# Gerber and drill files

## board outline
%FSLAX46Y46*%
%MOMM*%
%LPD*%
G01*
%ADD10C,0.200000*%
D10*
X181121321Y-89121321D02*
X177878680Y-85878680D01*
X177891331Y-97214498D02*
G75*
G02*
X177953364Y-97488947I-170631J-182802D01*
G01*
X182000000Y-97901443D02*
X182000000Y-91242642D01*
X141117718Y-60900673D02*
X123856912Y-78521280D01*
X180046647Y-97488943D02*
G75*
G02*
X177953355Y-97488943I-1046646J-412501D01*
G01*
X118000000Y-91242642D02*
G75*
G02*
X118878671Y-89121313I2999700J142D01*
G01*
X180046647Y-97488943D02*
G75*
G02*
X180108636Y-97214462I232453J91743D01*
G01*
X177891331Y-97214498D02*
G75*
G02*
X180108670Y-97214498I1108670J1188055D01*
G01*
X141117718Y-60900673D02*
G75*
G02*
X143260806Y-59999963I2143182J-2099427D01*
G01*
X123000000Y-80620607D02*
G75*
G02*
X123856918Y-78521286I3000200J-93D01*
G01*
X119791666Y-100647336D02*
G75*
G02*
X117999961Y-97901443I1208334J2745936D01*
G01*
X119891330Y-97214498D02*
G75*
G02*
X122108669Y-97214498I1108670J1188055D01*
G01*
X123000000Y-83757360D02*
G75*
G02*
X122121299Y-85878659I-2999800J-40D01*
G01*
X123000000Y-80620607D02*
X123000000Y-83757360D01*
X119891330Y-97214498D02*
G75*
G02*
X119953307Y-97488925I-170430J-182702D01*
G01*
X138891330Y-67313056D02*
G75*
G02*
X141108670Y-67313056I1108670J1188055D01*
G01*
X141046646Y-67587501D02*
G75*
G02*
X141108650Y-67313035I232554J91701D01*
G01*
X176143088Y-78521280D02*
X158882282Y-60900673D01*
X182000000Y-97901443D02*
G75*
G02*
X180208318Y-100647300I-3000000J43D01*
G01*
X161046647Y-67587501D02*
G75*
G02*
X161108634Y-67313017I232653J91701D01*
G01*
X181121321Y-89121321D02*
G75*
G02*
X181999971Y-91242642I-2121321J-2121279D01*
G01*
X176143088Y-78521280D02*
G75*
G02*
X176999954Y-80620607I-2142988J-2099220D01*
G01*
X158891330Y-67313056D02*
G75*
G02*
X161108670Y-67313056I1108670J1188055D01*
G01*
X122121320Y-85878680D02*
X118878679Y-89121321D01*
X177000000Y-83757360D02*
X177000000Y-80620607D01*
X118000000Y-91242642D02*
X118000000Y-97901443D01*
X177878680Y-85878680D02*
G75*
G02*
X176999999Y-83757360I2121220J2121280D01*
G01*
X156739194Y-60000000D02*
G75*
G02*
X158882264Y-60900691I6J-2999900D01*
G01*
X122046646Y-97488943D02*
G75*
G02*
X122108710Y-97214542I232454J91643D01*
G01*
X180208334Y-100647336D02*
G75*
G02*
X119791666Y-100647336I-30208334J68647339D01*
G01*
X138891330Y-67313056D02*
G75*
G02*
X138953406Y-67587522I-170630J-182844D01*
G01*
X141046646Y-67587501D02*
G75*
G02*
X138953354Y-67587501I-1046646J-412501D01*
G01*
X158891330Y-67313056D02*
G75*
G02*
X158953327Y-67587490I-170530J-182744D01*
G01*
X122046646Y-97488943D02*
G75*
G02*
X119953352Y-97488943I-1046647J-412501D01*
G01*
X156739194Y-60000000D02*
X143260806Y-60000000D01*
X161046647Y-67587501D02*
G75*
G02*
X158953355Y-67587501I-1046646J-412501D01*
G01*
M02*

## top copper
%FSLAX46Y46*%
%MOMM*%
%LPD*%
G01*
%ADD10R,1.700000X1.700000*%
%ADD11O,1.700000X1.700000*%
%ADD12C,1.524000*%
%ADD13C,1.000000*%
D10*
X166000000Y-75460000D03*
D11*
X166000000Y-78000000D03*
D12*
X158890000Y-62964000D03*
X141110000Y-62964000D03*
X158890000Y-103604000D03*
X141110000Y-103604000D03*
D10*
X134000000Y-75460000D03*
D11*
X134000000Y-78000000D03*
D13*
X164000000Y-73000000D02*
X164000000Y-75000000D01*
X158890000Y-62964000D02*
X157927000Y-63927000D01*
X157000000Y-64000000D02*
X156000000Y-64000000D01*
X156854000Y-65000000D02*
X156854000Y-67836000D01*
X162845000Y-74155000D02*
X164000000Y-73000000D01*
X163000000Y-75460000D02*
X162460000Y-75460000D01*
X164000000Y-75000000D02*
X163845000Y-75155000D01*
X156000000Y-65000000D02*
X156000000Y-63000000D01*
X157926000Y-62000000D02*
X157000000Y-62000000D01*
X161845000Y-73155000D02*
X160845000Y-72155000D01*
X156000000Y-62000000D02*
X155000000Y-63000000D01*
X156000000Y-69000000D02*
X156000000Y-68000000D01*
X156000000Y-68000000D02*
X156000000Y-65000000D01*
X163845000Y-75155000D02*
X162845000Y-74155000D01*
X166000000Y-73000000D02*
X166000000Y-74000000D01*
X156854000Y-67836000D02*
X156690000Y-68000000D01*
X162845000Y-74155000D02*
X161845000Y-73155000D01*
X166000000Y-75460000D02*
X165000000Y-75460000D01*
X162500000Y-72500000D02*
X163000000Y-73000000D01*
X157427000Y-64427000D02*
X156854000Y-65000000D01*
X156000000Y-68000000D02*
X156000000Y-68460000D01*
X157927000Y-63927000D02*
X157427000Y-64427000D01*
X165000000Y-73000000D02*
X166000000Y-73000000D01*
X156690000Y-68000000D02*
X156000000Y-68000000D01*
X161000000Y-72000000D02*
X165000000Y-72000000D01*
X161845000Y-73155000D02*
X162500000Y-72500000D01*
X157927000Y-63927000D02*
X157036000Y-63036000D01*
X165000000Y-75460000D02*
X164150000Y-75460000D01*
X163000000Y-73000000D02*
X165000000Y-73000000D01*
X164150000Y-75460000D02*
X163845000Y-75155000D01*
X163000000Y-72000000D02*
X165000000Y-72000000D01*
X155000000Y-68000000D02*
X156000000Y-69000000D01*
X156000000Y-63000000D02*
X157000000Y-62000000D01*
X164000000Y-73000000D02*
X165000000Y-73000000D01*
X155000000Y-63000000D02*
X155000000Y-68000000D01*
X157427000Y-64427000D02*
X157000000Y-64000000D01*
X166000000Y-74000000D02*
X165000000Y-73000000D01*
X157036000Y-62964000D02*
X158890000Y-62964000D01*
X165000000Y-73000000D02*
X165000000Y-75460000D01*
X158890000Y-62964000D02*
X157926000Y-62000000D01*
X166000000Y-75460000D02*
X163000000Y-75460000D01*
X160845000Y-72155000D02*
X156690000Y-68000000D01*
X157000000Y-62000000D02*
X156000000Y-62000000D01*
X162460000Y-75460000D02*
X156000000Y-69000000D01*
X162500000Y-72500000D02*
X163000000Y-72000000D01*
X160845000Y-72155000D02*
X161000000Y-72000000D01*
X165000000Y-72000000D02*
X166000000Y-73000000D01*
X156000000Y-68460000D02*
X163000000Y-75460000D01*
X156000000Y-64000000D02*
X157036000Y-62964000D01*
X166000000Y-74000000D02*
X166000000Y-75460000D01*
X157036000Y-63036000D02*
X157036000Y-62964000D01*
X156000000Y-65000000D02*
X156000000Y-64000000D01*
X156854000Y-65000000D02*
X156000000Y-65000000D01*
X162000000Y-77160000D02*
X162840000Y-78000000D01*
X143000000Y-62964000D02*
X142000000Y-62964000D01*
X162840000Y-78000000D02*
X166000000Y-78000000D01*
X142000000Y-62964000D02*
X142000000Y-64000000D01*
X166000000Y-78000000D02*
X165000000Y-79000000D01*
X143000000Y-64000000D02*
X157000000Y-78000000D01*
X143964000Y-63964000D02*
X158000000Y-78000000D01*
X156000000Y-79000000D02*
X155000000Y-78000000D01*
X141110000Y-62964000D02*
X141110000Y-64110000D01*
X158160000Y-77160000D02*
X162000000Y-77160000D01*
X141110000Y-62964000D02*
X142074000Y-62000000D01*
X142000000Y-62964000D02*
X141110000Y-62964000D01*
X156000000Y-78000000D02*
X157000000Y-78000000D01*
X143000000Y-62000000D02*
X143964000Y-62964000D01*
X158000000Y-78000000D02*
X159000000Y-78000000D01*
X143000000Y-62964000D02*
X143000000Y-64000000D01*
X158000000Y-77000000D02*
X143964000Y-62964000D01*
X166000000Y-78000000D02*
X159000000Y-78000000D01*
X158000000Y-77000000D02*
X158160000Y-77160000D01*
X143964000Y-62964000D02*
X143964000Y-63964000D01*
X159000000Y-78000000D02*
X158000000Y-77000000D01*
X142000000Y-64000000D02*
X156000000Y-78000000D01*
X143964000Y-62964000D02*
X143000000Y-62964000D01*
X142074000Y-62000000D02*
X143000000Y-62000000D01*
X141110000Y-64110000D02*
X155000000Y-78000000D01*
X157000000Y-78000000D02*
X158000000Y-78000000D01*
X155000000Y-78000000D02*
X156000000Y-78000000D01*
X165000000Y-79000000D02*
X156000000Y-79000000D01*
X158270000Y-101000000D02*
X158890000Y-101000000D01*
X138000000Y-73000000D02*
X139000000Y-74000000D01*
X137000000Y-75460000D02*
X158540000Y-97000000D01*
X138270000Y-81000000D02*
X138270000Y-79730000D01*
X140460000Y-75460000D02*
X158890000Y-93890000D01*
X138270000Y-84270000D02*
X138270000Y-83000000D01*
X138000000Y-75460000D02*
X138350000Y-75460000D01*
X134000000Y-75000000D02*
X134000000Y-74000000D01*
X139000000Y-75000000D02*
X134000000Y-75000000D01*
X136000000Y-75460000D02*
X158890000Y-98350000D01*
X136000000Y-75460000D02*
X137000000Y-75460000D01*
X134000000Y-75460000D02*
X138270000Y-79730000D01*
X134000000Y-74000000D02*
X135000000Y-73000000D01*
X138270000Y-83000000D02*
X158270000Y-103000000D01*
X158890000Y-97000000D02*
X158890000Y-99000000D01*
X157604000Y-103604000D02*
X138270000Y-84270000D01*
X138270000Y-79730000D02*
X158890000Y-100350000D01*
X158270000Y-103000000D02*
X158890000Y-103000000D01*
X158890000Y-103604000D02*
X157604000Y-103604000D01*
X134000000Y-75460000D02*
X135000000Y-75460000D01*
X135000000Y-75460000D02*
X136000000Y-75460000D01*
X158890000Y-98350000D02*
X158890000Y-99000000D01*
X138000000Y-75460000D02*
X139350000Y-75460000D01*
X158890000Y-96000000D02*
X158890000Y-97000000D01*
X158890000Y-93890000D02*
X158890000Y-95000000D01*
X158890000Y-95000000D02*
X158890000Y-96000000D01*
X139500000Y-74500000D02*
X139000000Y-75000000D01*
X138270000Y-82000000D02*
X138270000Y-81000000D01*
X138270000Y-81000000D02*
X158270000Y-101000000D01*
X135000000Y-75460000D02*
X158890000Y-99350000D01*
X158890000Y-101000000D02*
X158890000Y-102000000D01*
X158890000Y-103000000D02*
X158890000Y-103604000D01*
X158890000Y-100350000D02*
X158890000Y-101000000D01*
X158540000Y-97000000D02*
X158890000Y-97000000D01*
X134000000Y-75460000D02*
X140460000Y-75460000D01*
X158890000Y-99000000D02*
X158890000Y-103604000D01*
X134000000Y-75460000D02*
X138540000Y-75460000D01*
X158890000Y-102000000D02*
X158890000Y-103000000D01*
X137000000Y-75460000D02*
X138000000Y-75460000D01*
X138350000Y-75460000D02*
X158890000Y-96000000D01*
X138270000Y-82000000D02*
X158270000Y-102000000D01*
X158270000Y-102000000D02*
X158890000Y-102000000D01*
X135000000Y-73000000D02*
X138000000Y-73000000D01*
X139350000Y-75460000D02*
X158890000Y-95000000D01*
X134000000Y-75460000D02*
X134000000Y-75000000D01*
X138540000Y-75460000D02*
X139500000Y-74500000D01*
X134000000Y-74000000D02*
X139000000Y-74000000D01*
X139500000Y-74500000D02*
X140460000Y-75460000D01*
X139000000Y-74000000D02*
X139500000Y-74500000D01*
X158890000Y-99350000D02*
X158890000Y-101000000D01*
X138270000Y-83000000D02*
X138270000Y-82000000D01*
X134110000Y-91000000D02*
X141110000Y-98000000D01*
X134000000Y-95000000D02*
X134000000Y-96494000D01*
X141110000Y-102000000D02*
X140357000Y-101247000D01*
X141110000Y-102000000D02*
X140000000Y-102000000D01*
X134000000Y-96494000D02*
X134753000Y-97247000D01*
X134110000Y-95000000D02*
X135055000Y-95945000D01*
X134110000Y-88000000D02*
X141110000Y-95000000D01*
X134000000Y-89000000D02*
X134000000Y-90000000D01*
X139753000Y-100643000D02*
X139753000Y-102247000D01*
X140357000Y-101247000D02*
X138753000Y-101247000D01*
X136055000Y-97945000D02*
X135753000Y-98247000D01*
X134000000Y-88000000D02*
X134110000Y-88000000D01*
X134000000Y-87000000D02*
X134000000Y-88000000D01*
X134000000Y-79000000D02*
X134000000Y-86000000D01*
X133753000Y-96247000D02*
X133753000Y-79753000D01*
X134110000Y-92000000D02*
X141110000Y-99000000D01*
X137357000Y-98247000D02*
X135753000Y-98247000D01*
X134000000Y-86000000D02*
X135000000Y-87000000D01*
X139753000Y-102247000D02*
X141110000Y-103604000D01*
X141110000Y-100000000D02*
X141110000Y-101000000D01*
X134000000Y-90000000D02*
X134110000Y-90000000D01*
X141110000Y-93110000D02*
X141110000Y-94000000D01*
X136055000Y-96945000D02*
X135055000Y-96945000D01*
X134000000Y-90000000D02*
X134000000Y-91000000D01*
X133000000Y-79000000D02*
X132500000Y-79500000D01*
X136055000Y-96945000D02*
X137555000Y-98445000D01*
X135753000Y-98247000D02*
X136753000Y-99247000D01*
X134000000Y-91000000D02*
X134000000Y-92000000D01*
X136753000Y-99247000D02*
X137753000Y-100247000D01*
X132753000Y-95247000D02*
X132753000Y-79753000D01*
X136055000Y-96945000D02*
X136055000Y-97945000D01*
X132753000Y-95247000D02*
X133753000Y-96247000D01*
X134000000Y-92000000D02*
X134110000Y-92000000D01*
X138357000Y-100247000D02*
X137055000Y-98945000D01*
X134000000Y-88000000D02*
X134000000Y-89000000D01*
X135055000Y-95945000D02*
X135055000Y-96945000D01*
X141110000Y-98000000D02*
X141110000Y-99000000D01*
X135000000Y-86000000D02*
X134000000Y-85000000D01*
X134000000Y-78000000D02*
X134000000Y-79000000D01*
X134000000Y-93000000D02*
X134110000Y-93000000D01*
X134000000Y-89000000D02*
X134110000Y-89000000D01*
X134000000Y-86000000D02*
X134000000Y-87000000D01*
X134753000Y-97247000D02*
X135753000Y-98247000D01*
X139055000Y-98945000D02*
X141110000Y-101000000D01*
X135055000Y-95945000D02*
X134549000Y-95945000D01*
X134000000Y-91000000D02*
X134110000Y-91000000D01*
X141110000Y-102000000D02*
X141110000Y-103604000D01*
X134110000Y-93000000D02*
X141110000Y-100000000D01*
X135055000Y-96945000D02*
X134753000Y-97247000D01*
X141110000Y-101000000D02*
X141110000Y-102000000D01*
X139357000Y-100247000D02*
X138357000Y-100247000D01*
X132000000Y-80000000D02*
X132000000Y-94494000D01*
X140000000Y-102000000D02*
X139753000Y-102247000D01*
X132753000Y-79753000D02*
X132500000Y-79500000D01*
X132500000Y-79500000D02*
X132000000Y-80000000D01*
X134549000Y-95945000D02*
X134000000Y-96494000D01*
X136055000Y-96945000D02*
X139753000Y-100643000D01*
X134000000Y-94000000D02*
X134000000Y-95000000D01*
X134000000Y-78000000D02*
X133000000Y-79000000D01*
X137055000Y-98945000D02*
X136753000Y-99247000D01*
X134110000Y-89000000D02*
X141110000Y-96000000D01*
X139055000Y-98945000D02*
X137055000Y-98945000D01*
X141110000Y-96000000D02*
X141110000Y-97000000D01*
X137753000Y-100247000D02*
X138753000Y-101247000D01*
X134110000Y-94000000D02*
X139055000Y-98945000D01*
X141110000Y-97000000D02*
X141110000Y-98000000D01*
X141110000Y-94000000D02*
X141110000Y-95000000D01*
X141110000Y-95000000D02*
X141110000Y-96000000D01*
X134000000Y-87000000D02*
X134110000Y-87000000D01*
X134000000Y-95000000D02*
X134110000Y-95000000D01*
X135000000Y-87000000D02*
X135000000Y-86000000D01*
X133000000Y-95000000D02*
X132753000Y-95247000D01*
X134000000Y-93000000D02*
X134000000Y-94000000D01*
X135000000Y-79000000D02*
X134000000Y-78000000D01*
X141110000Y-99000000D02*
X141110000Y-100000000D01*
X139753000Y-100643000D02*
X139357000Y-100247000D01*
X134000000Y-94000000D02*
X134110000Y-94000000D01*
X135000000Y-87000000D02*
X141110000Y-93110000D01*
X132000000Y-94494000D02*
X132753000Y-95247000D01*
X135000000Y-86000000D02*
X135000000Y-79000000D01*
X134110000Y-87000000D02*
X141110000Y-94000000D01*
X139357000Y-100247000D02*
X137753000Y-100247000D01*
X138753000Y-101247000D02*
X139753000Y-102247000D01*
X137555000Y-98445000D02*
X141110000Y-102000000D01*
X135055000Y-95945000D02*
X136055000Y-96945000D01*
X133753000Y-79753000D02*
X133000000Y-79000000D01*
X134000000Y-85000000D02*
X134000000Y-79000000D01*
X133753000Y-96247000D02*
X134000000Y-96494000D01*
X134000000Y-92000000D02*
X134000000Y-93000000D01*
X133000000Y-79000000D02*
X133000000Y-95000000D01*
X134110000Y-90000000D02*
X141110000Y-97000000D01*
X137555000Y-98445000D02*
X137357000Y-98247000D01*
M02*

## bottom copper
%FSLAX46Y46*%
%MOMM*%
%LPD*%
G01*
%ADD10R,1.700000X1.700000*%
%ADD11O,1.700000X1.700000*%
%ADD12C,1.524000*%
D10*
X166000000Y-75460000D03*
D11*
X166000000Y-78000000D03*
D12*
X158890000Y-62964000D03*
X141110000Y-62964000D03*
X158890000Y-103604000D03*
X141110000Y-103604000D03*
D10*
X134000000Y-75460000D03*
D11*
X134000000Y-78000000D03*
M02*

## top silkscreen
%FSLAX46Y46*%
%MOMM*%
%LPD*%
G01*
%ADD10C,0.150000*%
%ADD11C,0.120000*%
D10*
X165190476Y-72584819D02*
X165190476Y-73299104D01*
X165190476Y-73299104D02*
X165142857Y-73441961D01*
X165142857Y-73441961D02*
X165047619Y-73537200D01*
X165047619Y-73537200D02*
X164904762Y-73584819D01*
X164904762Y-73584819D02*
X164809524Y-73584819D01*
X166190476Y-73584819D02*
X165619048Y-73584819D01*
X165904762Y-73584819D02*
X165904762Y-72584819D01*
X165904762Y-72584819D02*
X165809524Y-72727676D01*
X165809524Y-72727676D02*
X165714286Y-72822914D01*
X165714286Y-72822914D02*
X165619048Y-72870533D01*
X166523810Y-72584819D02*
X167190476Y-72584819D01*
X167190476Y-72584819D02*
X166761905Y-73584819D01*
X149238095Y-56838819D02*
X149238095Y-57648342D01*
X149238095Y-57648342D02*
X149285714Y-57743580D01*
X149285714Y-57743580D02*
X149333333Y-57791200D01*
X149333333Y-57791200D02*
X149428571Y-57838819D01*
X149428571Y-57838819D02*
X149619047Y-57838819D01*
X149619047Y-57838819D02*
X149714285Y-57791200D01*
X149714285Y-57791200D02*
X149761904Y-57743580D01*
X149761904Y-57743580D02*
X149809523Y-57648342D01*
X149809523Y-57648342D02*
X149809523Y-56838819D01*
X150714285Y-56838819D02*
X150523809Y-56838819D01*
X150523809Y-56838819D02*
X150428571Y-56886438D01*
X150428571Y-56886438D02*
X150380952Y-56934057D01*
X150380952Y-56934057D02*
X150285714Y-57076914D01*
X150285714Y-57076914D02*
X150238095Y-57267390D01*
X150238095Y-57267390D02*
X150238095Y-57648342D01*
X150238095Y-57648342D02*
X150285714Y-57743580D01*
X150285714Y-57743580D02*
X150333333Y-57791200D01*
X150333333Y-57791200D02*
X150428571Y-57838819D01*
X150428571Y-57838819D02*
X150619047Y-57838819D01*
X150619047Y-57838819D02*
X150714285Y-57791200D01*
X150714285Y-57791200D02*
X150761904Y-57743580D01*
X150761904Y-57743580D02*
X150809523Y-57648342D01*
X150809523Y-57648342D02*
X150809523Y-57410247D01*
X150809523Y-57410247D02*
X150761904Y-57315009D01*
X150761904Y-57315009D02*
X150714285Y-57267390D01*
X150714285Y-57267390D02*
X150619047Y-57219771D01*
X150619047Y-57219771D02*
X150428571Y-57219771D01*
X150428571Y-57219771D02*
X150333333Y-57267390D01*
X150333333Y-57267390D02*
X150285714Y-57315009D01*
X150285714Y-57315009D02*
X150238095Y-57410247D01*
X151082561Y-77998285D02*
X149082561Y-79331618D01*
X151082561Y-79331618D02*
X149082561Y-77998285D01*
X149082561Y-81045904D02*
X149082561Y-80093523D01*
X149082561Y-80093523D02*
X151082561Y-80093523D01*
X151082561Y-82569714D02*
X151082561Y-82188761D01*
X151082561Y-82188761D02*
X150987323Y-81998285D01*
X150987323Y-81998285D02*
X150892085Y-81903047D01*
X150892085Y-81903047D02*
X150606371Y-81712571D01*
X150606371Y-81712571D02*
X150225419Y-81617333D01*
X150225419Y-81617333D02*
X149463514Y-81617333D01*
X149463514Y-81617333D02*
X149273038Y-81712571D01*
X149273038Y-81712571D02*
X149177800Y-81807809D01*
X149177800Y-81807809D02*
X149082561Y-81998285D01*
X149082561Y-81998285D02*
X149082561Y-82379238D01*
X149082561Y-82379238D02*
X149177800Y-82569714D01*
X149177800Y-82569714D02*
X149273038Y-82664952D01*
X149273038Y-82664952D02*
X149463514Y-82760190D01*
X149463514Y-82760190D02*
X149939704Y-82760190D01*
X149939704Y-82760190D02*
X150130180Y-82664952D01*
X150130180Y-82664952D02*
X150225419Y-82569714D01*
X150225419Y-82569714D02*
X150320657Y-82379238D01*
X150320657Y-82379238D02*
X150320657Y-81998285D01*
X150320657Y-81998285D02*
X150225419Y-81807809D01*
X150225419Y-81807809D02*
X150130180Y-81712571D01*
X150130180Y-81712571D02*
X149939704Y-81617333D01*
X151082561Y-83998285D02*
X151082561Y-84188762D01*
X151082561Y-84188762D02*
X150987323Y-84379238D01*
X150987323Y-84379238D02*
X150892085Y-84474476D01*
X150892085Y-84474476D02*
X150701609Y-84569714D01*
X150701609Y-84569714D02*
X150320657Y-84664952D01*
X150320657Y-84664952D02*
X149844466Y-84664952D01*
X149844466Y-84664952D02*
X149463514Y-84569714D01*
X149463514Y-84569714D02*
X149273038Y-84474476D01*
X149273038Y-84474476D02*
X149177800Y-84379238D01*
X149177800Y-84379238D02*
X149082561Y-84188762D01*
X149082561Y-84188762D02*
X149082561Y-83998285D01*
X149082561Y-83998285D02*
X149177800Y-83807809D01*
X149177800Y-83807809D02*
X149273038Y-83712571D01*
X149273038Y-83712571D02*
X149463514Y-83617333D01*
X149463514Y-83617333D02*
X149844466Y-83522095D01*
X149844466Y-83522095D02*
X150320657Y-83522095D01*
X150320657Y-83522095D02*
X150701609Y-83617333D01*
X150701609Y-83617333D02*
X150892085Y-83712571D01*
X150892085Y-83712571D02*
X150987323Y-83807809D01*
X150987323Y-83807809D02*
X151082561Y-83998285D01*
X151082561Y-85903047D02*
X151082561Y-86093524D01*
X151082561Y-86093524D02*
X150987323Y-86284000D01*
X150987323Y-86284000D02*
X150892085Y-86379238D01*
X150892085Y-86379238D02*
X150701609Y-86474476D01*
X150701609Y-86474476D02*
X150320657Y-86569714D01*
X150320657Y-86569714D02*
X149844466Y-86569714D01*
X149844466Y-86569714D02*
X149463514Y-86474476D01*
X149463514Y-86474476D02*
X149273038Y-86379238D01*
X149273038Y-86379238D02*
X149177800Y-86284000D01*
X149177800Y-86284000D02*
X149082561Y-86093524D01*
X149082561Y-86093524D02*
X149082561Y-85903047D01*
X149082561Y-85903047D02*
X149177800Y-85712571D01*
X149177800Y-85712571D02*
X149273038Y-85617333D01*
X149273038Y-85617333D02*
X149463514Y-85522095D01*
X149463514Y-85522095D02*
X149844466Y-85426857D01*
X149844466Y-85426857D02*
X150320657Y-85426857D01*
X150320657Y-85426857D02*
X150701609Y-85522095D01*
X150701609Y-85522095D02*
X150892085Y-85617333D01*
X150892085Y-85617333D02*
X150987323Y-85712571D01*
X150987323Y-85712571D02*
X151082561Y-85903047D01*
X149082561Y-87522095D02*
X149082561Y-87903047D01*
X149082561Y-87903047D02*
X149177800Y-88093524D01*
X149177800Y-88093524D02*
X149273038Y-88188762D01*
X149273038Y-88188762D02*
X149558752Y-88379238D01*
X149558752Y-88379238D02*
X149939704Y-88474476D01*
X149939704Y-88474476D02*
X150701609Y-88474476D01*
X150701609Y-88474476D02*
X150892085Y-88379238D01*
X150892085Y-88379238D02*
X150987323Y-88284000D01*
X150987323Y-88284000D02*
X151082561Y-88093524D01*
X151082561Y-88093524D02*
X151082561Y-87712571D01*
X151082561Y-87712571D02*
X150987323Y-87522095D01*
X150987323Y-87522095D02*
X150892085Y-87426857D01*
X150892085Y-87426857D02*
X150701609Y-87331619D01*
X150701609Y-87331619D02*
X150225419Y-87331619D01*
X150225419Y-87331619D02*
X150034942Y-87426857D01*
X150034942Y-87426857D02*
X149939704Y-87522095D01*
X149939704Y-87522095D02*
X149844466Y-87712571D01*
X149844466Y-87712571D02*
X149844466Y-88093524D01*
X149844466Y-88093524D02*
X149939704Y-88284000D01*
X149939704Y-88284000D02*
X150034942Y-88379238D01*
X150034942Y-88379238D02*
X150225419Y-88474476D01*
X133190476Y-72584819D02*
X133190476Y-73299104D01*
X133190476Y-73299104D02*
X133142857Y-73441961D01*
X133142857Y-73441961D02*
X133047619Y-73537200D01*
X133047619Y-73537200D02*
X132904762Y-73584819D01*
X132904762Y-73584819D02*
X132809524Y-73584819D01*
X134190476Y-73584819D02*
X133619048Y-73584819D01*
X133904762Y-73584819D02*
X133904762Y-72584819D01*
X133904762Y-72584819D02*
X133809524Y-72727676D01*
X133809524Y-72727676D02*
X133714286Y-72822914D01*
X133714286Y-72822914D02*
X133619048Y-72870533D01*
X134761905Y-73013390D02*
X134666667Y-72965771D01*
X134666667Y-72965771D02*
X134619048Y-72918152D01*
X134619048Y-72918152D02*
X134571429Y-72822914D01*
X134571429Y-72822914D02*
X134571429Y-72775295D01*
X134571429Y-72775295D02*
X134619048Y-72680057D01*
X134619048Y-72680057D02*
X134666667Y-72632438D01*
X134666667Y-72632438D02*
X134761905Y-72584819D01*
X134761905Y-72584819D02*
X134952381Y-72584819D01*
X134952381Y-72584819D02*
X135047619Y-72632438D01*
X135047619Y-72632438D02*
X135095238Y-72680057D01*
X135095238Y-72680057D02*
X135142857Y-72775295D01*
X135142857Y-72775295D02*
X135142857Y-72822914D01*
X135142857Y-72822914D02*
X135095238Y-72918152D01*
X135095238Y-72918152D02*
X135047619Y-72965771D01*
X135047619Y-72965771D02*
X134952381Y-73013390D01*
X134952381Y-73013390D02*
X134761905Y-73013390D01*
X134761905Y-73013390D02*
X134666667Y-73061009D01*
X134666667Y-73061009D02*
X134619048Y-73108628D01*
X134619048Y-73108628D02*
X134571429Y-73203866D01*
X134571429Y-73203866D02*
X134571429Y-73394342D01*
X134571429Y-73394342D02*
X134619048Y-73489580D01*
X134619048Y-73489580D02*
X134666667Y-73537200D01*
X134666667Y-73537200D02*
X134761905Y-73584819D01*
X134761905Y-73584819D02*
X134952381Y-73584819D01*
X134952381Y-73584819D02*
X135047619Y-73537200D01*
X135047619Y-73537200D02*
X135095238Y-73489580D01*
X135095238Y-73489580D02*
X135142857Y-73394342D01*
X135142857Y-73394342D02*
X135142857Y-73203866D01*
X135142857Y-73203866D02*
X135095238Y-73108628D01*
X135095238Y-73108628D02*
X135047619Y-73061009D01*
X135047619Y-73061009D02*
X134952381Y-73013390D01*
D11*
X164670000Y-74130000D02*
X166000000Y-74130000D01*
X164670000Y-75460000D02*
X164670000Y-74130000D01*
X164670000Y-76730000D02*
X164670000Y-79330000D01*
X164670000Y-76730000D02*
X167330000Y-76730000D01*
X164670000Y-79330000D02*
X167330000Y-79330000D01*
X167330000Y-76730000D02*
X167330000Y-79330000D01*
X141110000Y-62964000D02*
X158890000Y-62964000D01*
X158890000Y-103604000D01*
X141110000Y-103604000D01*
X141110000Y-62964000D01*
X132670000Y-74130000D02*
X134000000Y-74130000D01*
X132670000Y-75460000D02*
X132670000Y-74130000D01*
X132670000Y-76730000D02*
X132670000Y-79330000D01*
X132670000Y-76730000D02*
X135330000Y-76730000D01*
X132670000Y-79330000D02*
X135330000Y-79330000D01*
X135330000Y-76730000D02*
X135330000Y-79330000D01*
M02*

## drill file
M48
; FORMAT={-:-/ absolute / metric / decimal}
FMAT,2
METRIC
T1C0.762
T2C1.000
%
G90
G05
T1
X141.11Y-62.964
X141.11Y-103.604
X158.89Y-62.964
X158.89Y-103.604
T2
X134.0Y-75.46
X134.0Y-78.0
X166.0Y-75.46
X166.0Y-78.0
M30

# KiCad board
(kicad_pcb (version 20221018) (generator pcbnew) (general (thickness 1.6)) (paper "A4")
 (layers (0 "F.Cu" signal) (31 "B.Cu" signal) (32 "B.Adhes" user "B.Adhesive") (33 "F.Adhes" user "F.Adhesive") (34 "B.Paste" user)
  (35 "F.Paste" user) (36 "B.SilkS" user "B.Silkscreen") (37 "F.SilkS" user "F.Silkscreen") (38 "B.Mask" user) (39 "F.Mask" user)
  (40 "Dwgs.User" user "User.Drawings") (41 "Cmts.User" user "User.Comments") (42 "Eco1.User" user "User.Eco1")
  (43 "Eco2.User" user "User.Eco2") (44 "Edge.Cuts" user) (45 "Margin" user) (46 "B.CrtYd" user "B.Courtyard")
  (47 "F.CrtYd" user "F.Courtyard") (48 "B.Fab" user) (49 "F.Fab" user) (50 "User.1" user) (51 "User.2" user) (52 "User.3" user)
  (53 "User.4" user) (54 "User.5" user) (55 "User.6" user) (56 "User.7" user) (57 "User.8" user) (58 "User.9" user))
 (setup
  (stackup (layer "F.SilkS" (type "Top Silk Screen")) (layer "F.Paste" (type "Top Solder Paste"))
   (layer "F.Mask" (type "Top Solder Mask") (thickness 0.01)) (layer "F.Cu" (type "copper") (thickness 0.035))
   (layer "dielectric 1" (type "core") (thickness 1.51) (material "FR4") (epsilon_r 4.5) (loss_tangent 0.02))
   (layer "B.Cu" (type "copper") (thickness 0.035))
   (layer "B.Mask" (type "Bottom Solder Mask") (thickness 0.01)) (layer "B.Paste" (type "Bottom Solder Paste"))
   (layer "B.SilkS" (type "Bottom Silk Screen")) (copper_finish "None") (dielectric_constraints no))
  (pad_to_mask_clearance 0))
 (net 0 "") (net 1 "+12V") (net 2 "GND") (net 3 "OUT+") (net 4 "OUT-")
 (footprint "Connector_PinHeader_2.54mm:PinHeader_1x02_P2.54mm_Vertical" (layer "F.Cu") (at 166 75.46)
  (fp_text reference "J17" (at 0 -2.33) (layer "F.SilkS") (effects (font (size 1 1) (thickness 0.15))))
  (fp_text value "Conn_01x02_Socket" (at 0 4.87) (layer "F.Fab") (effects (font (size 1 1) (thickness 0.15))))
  (fp_line (start -1.33 -1.33) (end 0 -1.33) (stroke (width 0.12) (type solid)) (layer "F.SilkS"))
  (fp_line (start -1.33 0) (end -1.33 -1.33) (stroke (width 0.12) (type solid)) (layer "F.SilkS"))
  (fp_line (start -1.33 1.27) (end -1.33 3.87) (stroke (width 0.12) (type solid)) (layer "F.SilkS"))
  (fp_line (start -1.33 1.27) (end 1.33 1.27) (stroke (width 0.12) (type solid)) (layer "F.SilkS"))
  (fp_line (start -1.33 3.87) (end 1.33 3.87) (stroke (width 0.12) (type solid)) (layer "F.SilkS"))
  (fp_line (start 1.33 1.27) (end 1.33 3.87) (stroke (width 0.12) (type solid)) (layer "F.SilkS"))
  (pad "1" thru_hole rect (at 0 0) (size 1.7 1.7) (drill 1) (layers "*.Cu" "*.Mask") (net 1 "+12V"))
  (pad "2" thru_hole oval (at 0 2.54) (size 1.7 1.7) (drill 1) (layers "*.Cu" "*.Mask") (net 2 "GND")))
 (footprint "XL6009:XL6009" (layer "F.Cu") (at 150 57.884)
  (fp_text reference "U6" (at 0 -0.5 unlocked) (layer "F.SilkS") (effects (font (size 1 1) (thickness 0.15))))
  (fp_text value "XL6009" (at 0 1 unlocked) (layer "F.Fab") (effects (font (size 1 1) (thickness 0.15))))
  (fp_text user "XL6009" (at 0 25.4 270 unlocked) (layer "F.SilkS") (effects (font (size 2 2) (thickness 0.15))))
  (fp_rect (start -8.89 5.08) (end 8.89 45.72) (stroke (width 0.12) (type solid)) (fill none) (layer "F.SilkS"))
  (pad "1" thru_hole circle (at 8.89 5.08) (size 1.524 1.524) (drill 0.762) (layers "*.Cu" "*.Mask") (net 1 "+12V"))
  (pad "2" thru_hole circle (at -8.89 5.08) (size 1.524 1.524) (drill 0.762) (layers "*.Cu" "*.Mask") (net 2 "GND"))
  (pad "3" thru_hole circle (at 8.89 45.72) (size 1.524 1.524) (drill 0.762) (layers "*.Cu" "*.Mask") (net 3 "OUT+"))
  (pad "4" thru_hole circle (at -8.89 45.72) (size 1.524 1.524) (drill 0.762) (layers "*.Cu" "*.Mask") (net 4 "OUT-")))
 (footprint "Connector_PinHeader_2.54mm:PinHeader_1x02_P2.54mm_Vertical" (layer "F.Cu") (at 134 75.46)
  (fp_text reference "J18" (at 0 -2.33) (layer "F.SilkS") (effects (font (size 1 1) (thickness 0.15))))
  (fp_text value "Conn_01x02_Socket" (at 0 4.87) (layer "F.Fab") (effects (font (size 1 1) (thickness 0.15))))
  (fp_line (start -1.33 -1.33) (end 0 -1.33) (stroke (width 0.12) (type solid)) (layer "F.SilkS"))
  (fp_line (start -1.33 0) (end -1.33 -1.33) (stroke (width 0.12) (type solid)) (layer "F.SilkS"))
  (fp_line (start -1.33 1.27) (end -1.33 3.87) (stroke (width 0.12) (type solid)) (layer "F.SilkS"))
  (fp_line (start -1.33 1.27) (end 1.33 1.27) (stroke (width 0.12) (type solid)) (layer "F.SilkS"))
  (fp_line (start -1.33 3.87) (end 1.33 3.87) (stroke (width 0.12) (type solid)) (layer "F.SilkS"))
  (fp_line (start 1.33 1.27) (end 1.33 3.87) (stroke (width 0.12) (type solid)) (layer "F.SilkS"))
  (pad "1" thru_hole rect (at 0 0) (size 1.7 1.7) (drill 1) (layers "*.Cu" "*.Mask") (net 3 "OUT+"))
  (pad "2" thru_hole oval (at 0 2.54) (size 1.7 1.7) (drill 1) (layers "*.Cu" "*.Mask") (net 4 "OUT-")))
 (gr_line (start 181.121321 89.121321) (end 177.87868 85.87868) (stroke (width 0.2) (type solid)) (layer "Edge.Cuts"))
 (gr_arc (start 177.891331 97.214498) (mid 177.964609 97.342164) (end 177.953354 97.488943) (stroke (width 0.2) (type solid))
  (layer "Edge.Cuts"))
 (gr_line (start 182 97.901443) (end 182 91.242642) (stroke (width 0.2) (type solid)) (layer "Edge.Cuts"))
 (gr_line (start 141.117718 60.900673) (end 123.856912 78.52128) (stroke (width 0.2) (type solid)) (layer "Edge.Cuts"))
 (gr_arc (start 180.046647 97.488943) (mid 179 99.026444) (end 177.953354 97.488943) (stroke (width 0.2) (type solid)) (layer "Edge.Cuts"))
 (gr_arc (start 118 91.242642) (mid 118.228341 90.094582) (end 118.878679 89.121321) (stroke (width 0.2) (type solid)) (layer "Edge.Cuts"))
 (gr_arc (start 180.046647 97.488943) (mid 180.035365 97.342158) (end 180.10867 97.214498) (stroke (width 0.2) (type solid))
  (layer "Edge.Cuts"))
 (gr_arc (start 177.891331 97.214498) (mid 179 94.401444) (end 180.10867 97.214498) (stroke (width 0.2) (type solid)) (layer "Edge.Cuts"))
 (gr_arc (start 141.117718 60.900673) (mid 142.09848 60.23433) (end 143.260806 60) (stroke (width 0.2) (type solid)) (layer "Edge.Cuts"))
 (gr_arc (start 123 80.620607) (mid 123.222489 79.486874) (end 123.856912 78.52128) (stroke (width 0.2) (type solid)) (layer "Edge.Cuts"))
 (gr_arc (start 119.791666 100.647336) (mid 118.487531 99.540802) (end 118 97.901443) (stroke (width 0.2) (type solid)) (layer "Edge.Cuts"))
 (gr_arc (start 119.89133 97.214498) (mid 120.999999 94.401444) (end 122.108669 97.214498) (stroke (width 0.2) (type solid))
  (layer "Edge.Cuts"))
 (gr_arc (start 123 83.75736) (mid 122.771654 84.905417) (end 122.12132 85.87868) (stroke (width 0.2) (type solid)) (layer "Edge.Cuts"))
 (gr_line (start 123 80.620607) (end 123 83.75736) (stroke (width 0.2) (type solid)) (layer "Edge.Cuts"))
 (gr_arc (start 119.89133 97.214498) (mid 119.964638 97.342161) (end 119.953353 97.488943) (stroke (width 0.2) (type solid))
  (layer "Edge.Cuts"))
 (gr_arc (start 138.89133 67.313056) (mid 140 64.500001) (end 141.10867 67.313056) (stroke (width 0.2) (type solid)) (layer "Edge.Cuts"))
 (gr_arc (start 141.046646 67.587501) (mid 141.035382 67.440731) (end 141.10867 67.313056) (stroke (width 0.2) (type solid))
  (layer "Edge.Cuts"))
 (gr_line (start 176.143088 78.52128) (end 158.882282 60.900673) (stroke (width 0.2) (type solid)) (layer "Edge.Cuts"))
 (gr_arc (start 182 97.901443) (mid 181.512469 99.540802) (end 180.208334 100.647336) (stroke (width 0.2) (type solid)) (layer "Edge.Cuts"))
 (gr_arc (start 161.046647 67.587501) (mid 161.035388 67.440729) (end 161.10867 67.313056) (stroke (width 0.2) (type solid))
  (layer "Edge.Cuts"))
 (gr_arc (start 181.121321 89.121321) (mid 181.77164 90.094591) (end 182 91.242642) (stroke (width 0.2) (type solid)) (layer "Edge.Cuts"))
 (gr_arc (start 176.143088 78.52128) (mid 176.777534 79.486864) (end 177 80.620607) (stroke (width 0.2) (type solid)) (layer "Edge.Cuts"))
 (gr_arc (start 158.89133 67.313056) (mid 160 64.500001) (end 161.10867 67.313056) (stroke (width 0.2) (type solid)) (layer "Edge.Cuts"))
 (gr_line (start 122.12132 85.87868) (end 118.878679 89.121321) (stroke (width 0.2) (type solid)) (layer "Edge.Cuts"))
 (gr_line (start 177 83.75736) (end 177 80.620607) (stroke (width 0.2) (type solid)) (layer "Edge.Cuts"))
 (gr_line (start 118 91.242642) (end 118 97.901443) (stroke (width 0.2) (type solid)) (layer "Edge.Cuts"))
 (gr_arc (start 177.87868 85.87868) (mid 177.228356 84.905411) (end 177 83.75736) (stroke (width 0.2) (type solid)) (layer "Edge.Cuts"))
 (gr_arc (start 156.739194 60) (mid 157.901527 60.234315) (end 158.882282 60.900673) (stroke (width 0.2) (type solid)) (layer "Edge.Cuts"))
 (gr_arc (start 122.046646 97.488943) (mid 122.035369 97.342155) (end 122.108669 97.214498) (stroke (width 0.2) (type solid))
  (layer "Edge.Cuts"))
 (gr_arc (start 180.208334 100.647336) (mid 150 107.000001) (end 119.791666 100.647336) (stroke (width 0.2) (type solid))
  (layer "Edge.Cuts"))
 (gr_arc (start 138.89133 67.313056) (mid 138.964601 67.440727) (end 138.953353 67.587501) (stroke (width 0.2) (type solid))
  (layer "Edge.Cuts"))
 (gr_arc (start 141.046646 67.587501) (mid 139.999999 69.125003) (end 138.953353 67.587501) (stroke (width 0.2) (type solid))
  (layer "Edge.Cuts"))
 (gr_arc (start 158.89133 67.313056) (mid 158.964631 67.440724) (end 158.953354 67.587501) (stroke (width 0.2) (type solid))
  (layer "Edge.Cuts"))
 (gr_arc (start 122.046646 97.488943) (mid 120.999999 99.026445) (end 119.953353 97.488943) (stroke (width 0.2) (type solid))
  (layer "Edge.Cuts"))
 (gr_line (start 156.739194 60) (end 143.260806 60) (stroke (width 0.2) (type solid)) (layer "Edge.Cuts"))
 (gr_arc (start 161.046647 67.587501) (mid 160 69.125002) (end 158.953354 67.587501) (stroke (width 0.2) (type solid)) (layer "Edge.Cuts"))
 (segment (start 164 73) (end 164 75) (width 1) (layer "F.Cu") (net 1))
 (segment (start 158.89 62.964) (end 157.927 63.927) (width 1) (layer "F.Cu") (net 1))
 (segment (start 157 64) (end 156 64) (width 1) (layer "F.Cu") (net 1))
 (segment (start 156.854 65) (end 156.854 67.836) (width 1) (layer "F.Cu") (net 1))
 (segment (start 162.845 74.155) (end 164 73) (width 1) (layer "F.Cu") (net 1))
 (segment (start 163 75.46) (end 162.46 75.46) (width 1) (layer "F.Cu") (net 1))
 (segment (start 164 75) (end 163.845 75.155) (width 1) (layer "F.Cu") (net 1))
 (segment (start 156 65) (end 156 63) (width 1) (layer "F.Cu") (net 1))
 (segment (start 157.926 62) (end 157 62) (width 1) (layer "F.Cu") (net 1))
 (segment (start 161.845 73.155) (end 160.845 72.155) (width 1) (layer "F.Cu") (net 1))
 (segment (start 156 62) (end 155 63) (width 1) (layer "F.Cu") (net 1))
 (segment (start 156 69) (end 156 68) (width 1) (layer "F.Cu") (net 1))
 (segment (start 156 68) (end 156 65) (width 1) (layer "F.Cu") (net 1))
 (segment (start 163.845 75.155) (end 162.845 74.155) (width 1) (layer "F.Cu") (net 1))
 (segment (start 166 73) (end 166 74) (width 1) (layer "F.Cu") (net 1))
 (segment (start 156.854 67.836) (end 156.69 68) (width 1) (layer "F.Cu") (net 1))
 (segment (start 162.845 74.155) (end 161.845 73.155) (width 1) (layer "F.Cu") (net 1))
 (segment (start 166 75.46) (end 165 75.46) (width 1) (layer "F.Cu") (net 1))
 (segment (start 162.5 72.5) (end 163 73) (width 1) (layer "F.Cu") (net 1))
 (segment (start 157.427 64.427) (end 156.854 65) (width 1) (layer "F.Cu") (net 1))
 (segment (start 156 68) (end 156 68.46) (width 1) (layer "F.Cu") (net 1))
 (segment (start 157.927 63.927) (end 157.427 64.427) (width 1) (layer "F.Cu") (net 1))
 (segment (start 165 73) (end 166 73) (width 1) (layer "F.Cu") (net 1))
 (segment (start 156.69 68) (end 156 68) (width 1) (layer "F.Cu") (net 1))
 (segment (start 161 72) (end 165 72) (width 1) (layer "F.Cu") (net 1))
 (segment (start 161.845 73.155) (end 162.5 72.5) (width 1) (layer "F.Cu") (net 1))
 (segment (start 157.927 63.927) (end 157.036 63.036) (width 1) (layer "F.Cu") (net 1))
 (segment (start 165 75.46) (end 164.15 75.46) (width 1) (layer "F.Cu") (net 1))
 (segment (start 163 73) (end 165 73) (width 1) (layer "F.Cu") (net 1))
 (segment (start 164.15 75.46) (end 163.845 75.155) (width 1) (layer "F.Cu") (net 1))
 (segment (start 163 72) (end 165 72) (width 1) (layer "F.Cu") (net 1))
 (segment (start 155 68) (end 156 69) (width 1) (layer "F.Cu") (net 1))
 (segment (start 156 63) (end 157 62) (width 1) (layer "F.Cu") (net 1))
 (segment (start 164 73) (end 165 73) (width 1) (layer "F.Cu") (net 1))
 (segment (start 155 63) (end 155 68) (width 1) (layer "F.Cu") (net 1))
 (segment (start 157.427 64.427) (end 157 64) (width 1) (layer "F.Cu") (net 1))
 (segment (start 166 74) (end 165 73) (width 1) (layer "F.Cu") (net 1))
 (segment (start 157.036 62.964) (end 158.89 62.964) (width 1) (layer "F.Cu") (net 1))
 (segment (start 165 73) (end 165 75.46) (width 1) (layer "F.Cu") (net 1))
 (segment (start 158.89 62.964) (end 157.926 62) (width 1) (layer "F.Cu") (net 1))
 (segment (start 166 75.46) (end 163 75.46) (width 1) (layer "F.Cu") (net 1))
 (segment (start 160.845 72.155) (end 156.69 68) (width 1) (layer "F.Cu") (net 1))
 (segment (start 157 62) (end 156 62) (width 1) (layer "F.Cu") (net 1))
 (segment (start 162.46 75.46) (end 156 69) (width 1) (layer "F.Cu") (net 1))
 (segment (start 162.5 72.5) (end 163 72) (width 1) (layer "F.Cu") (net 1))
 (segment (start 160.845 72.155) (end 161 72) (width 1) (layer "F.Cu") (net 1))
 (segment (start 165 72) (end 166 73) (width 1) (layer "F.Cu") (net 1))
 (segment (start 156 68.46) (end 163 75.46) (width 1) (layer "F.Cu") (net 1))
 (segment (start 156 64) (end 157.036 62.964) (width 1) (layer "F.Cu") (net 1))
 (segment (start 166 74) (end 166 75.46) (width 1) (layer "F.Cu") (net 1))
 (segment (start 157.036 63.036) (end 157.036 62.964) (width 1) (layer "F.Cu") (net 1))
 (segment (start 156 65) (end 156 64) (width 1) (layer "F.Cu") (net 1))
 (segment (start 156.854 65) (end 156 65) (width 1) (layer "F.Cu") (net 1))
 (segment (start 162 77.16) (end 162.84 78) (width 1) (layer "F.Cu") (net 2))
 (segment (start 143 62.964) (end 142 62.964) (width 1) (layer "F.Cu") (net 2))
 (segment (start 162.84 78) (end 166 78) (width 1) (layer "F.Cu") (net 2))
 (segment (start 142 62.964) (end 142 64) (width 1) (layer "F.Cu") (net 2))
 (segment (start 166 78) (end 165 79) (width 1) (layer "F.Cu") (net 2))
 (segment (start 143 64) (end 157 78) (width 1) (layer "F.Cu") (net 2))
 (segment (start 143.964 63.964) (end 158 78) (width 1) (layer "F.Cu") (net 2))
 (segment (start 156 79) (end 155 78) (width 1) (layer "F.Cu") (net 2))
 (segment (start 141.11 62.964) (end 141.11 64.11) (width 1) (layer "F.Cu") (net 2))
 (segment (start 158.16 77.16) (end 162 77.16) (width 1) (layer "F.Cu") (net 2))
 (segment (start 141.11 62.964) (end 142.074 62) (width 1) (layer "F.Cu") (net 2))
 (segment (start 142 62.964) (end 141.11 62.964) (width 1) (layer "F.Cu") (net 2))
 (segment (start 156 78) (end 157 78) (width 1) (layer "F.Cu") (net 2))
 (segment (start 143 62) (end 143.964 62.964) (width 1) (layer "F.Cu") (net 2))
 (segment (start 158 78) (end 159 78) (width 1) (layer "F.Cu") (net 2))
 (segment (start 143 62.964) (end 143 64) (width 1) (layer "F.Cu") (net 2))
 (segment (start 158 77) (end 143.964 62.964) (width 1) (layer "F.Cu") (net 2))
 (segment (start 166 78) (end 159 78) (width 1) (layer "F.Cu") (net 2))
 (segment (start 158 77) (end 158.16 77.16) (width 1) (layer "F.Cu") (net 2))
 (segment (start 143.964 62.964) (end 143.964 63.964) (width 1) (layer "F.Cu") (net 2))
 (segment (start 159 78) (end 158 77) (width 1) (layer "F.Cu") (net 2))
 (segment (start 142 64) (end 156 78) (width 1) (layer "F.Cu") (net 2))
 (segment (start 143.964 62.964) (end 143 62.964) (width 1) (layer "F.Cu") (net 2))
 (segment (start 142.074 62) (end 143 62) (width 1) (layer "F.Cu") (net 2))
 (segment (start 141.11 64.11) (end 155 78) (width 1) (layer "F.Cu") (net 2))
 (segment (start 157 78) (end 158 78) (width 1) (layer "F.Cu") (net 2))
 (segment (start 155 78) (end 156 78) (width 1) (layer "F.Cu") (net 2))
 (segment (start 165 79) (end 156 79) (width 1) (layer "F.Cu") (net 2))
 (segment (start 158.27 101) (end 158.89 101) (width 1) (layer "F.Cu") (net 3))
 (segment (start 138 73) (end 139 74) (width 1) (layer "F.Cu") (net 3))
 (segment (start 137 75.46) (end 158.54 97) (width 1) (layer "F.Cu") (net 3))
 (segment (start 138.27 81) (end 138.27 79.73) (width 1) (layer "F.Cu") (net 3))
 (segment (start 140.46 75.46) (end 158.89 93.89) (width 1) (layer "F.Cu") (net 3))
 (segment (start 138.27 84.27) (end 138.27 83) (width 1) (layer "F.Cu") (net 3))
 (segment (start 138 75.46) (end 138.35 75.46) (width 1) (layer "F.Cu") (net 3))
 (segment (start 134 75) (end 134 74) (width 1) (layer "F.Cu") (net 3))
 (segment (start 139 75) (end 134 75) (width 1) (layer "F.Cu") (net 3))
 (segment (start 136 75.46) (end 158.89 98.35) (width 1) (layer "F.Cu") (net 3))
 (segment (start 136 75.46) (end 137 75.46) (width 1) (layer "F.Cu") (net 3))
 (segment (start 134 75.46) (end 138.27 79.73) (width 1) (layer "F.Cu") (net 3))
 (segment (start 134 74) (end 135 73) (width 1) (layer "F.Cu") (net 3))
 (segment (start 138.27 83) (end 158.27 103) (width 1) (layer "F.Cu") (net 3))
 (segment (start 158.89 97) (end 158.89 99) (width 1) (layer "F.Cu") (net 3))
 (segment (start 157.604 103.604) (end 138.27 84.27) (width 1) (layer "F.Cu") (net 3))
 (segment (start 138.27 79.73) (end 158.89 100.35) (width 1) (layer "F.Cu") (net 3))
 (segment (start 158.27 103) (end 158.89 103) (width 1) (layer "F.Cu") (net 3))
 (segment (start 158.89 103.604) (end 157.604 103.604) (width 1) (layer "F.Cu") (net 3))
 (segment (start 134 75.46) (end 135 75.46) (width 1) (layer "F.Cu") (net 3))
 (segment (start 135 75.46) (end 136 75.46) (width 1) (layer "F.Cu") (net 3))
 (segment (start 158.89 98.35) (end 158.89 99) (width 1) (layer "F.Cu") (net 3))
 (segment (start 138 75.46) (end 139.35 75.46) (width 1) (layer "F.Cu") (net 3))
 (segment (start 158.89 96) (end 158.89 97) (width 1) (layer "F.Cu") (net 3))
 (segment (start 158.89 93.89) (end 158.89 95) (width 1) (layer "F.Cu") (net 3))
 (segment (start 158.89 95) (end 158.89 96) (width 1) (layer "F.Cu") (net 3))
 (segment (start 139.5 74.5) (end 139 75) (width 1) (layer "F.Cu") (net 3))
 (segment (start 138.27 82) (end 138.27 81) (width 1) (layer "F.Cu") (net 3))
 (segment (start 138.27 81) (end 158.27 101) (width 1) (layer "F.Cu") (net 3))
 (segment (start 135 75.46) (end 158.89 99.35) (width 1) (layer "F.Cu") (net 3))
 (segment (start 158.89 101) (end 158.89 102) (width 1) (layer "F.Cu") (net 3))
 (segment (start 158.89 103) (end 158.89 103.604) (width 1) (layer "F.Cu") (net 3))
 (segment (start 158.89 100.35) (end 158.89 101) (width 1) (layer "F.Cu") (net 3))
 (segment (start 158.54 97) (end 158.89 97) (width 1) (layer "F.Cu") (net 3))
 (segment (start 134 75.46) (end 140.46 75.46) (width 1) (layer "F.Cu") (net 3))
 (segment (start 158.89 99) (end 158.89 103.604) (width 1) (layer "F.Cu") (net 3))
 (segment (start 134 75.46) (end 138.54 75.46) (width 1) (layer "F.Cu") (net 3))
 (segment (start 158.89 102) (end 158.89 103) (width 1) (layer "F.Cu") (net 3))
 (segment (start 137 75.46) (end 138 75.46) (width 1) (layer "F.Cu") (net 3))
 (segment (start 138.35 75.46) (end 158.89 96) (width 1) (layer "F.Cu") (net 3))
 (segment (start 138.27 82) (end 158.27 102) (width 1) (layer "F.Cu") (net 3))
 (segment (start 158.27 102) (end 158.89 102) (width 1) (layer "F.Cu") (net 3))
 (segment (start 135 73) (end 138 73) (width 1) (layer "F.Cu") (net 3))
 (segment (start 139.35 75.46) (end 158.89 95) (width 1) (layer "F.Cu") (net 3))
 (segment (start 134 75.46) (end 134 75) (width 1) (layer "F.Cu") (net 3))
 (segment (start 138.54 75.46) (end 139.5 74.5) (width 1) (layer "F.Cu") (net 3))
 (segment (start 134 74) (end 139 74) (width 1) (layer "F.Cu") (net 3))
 (segment (start 139.5 74.5) (end 140.46 75.46) (width 1) (layer "F.Cu") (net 3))
 (segment (start 139 74) (end 139.5 74.5) (width 1) (layer "F.Cu") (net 3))
 (segment (start 158.89 99.35) (end 158.89 101) (width 1) (layer "F.Cu") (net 3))
 (segment (start 138.27 83) (end 138.27 82) (width 1) (layer "F.Cu") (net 3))
 (segment (start 134.11 91) (end 141.11 98) (width 1) (layer "F.Cu") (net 4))
 (segment (start 134 95) (end 134 96.494) (width 1) (layer "F.Cu") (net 4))
 (segment (start 141.11 102) (end 140.357 101.247) (width 1) (layer "F.Cu") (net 4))
 (segment (start 141.11 102) (end 140 102) (width 1) (layer "F.Cu") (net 4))
 (segment (start 134 96.494) (end 134.753 97.247) (width 1) (layer "F.Cu") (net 4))
 (segment (start 134.11 95) (end 135.055 95.945) (width 1) (layer "F.Cu") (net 4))
 (segment (start 134.11 88) (end 141.11 95) (width 1) (layer "F.Cu") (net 4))
 (segment (start 134 89) (end 134 90) (width 1) (layer "F.Cu") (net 4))
 (segment (start 139.753 100.643) (end 139.753 102.247) (width 1) (layer "F.Cu") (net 4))
 (segment (start 140.357 101.247) (end 138.753 101.247) (width 1) (layer "F.Cu") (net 4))
 (segment (start 136.055 97.945) (end 135.753 98.247) (width 1) (layer "F.Cu") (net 4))
 (segment (start 134 88) (end 134.11 88) (width 1) (layer "F.Cu") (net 4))
 (segment (start 134 87) (end 134 88) (width 1) (layer "F.Cu") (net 4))
 (segment (start 134 79) (end 134 86) (width 1) (layer "F.Cu") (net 4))
 (segment (start 133.753 96.247) (end 133.753 79.753) (width 1) (layer "F.Cu") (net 4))
 (segment (start 134.11 92) (end 141.11 99) (width 1) (layer "F.Cu") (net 4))
 (segment (start 137.357 98.247) (end 135.753 98.247) (width 1) (layer "F.Cu") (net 4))
 (segment (start 134 86) (end 135 87) (width 1) (layer "F.Cu") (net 4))
 (segment (start 139.753 102.247) (end 141.11 103.604) (width 1) (layer "F.Cu") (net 4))
 (segment (start 141.11 100) (end 141.11 101) (width 1) (layer "F.Cu") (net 4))
 (segment (start 134 90) (end 134.11 90) (width 1) (layer "F.Cu") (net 4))
 (segment (start 141.11 93.11) (end 141.11 94) (width 1) (layer "F.Cu") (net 4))
 (segment (start 136.055 96.945) (end 135.055 96.945) (width 1) (layer "F.Cu") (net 4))
 (segment (start 134 90) (end 134 91) (width 1) (layer "F.Cu") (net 4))
 (segment (start 133 79) (end 132.5 79.5) (width 1) (layer "F.Cu") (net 4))
 (segment (start 136.055 96.945) (end 137.555 98.445) (width 1) (layer "F.Cu") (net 4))
 (segment (start 135.753 98.247) (end 136.753 99.247) (width 1) (layer "F.Cu") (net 4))
 (segment (start 134 91) (end 134 92) (width 1) (layer "F.Cu") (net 4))
 (segment (start 136.753 99.247) (end 137.753 100.247) (width 1) (layer "F.Cu") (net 4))
 (segment (start 132.753 95.247) (end 132.753 79.753) (width 1) (layer "F.Cu") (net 4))
 (segment (start 136.055 96.945) (end 136.055 97.945) (width 1) (layer "F.Cu") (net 4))
 (segment (start 132.753 95.247) (end 133.753 96.247) (width 1) (layer "F.Cu") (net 4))
 (segment (start 134 92) (end 134.11 92) (width 1) (layer "F.Cu") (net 4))
 (segment (start 138.357 100.247) (end 137.055 98.945) (width 1) (layer "F.Cu") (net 4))
 (segment (start 134 88) (end 134 89) (width 1) (layer "F.Cu") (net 4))
 (segment (start 135.055 95.945) (end 135.055 96.945) (width 1) (layer "F.Cu") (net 4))
 (segment (start 141.11 98) (end 141.11 99) (width 1) (layer "F.Cu") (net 4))
 (segment (start 135 86) (end 134 85) (width 1) (layer "F.Cu") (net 4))
 (segment (start 134 78) (end 134 79) (width 1) (layer "F.Cu") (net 4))
 (segment (start 134 93) (end 134.11 93) (width 1) (layer "F.Cu") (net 4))
 (segment (start 134 89) (end 134.11 89) (width 1) (layer "F.Cu") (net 4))
 (segment (start 134 86) (end 134 87) (width 1) (layer "F.Cu") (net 4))
 (segment (start 134.753 97.247) (end 135.753 98.247) (width 1) (layer "F.Cu") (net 4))
 (segment (start 139.055 98.945) (end 141.11 101) (width 1) (layer "F.Cu") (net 4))
 (segment (start 135.055 95.945) (end 134.549 95.945) (width 1) (layer "F.Cu") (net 4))
 (segment (start 134 91) (end 134.11 91) (width 1) (layer "F.Cu") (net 4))
 (segment (start 141.11 102) (end 141.11 103.604) (width 1) (layer "F.Cu") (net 4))
 (segment (start 134.11 93) (end 141.11 100) (width 1) (layer "F.Cu") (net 4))
 (segment (start 135.055 96.945) (end 134.753 97.247) (width 1) (layer "F.Cu") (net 4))
 (segment (start 141.11 101) (end 141.11 102) (width 1) (layer "F.Cu") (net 4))
 (segment (start 139.357 100.247) (end 138.357 100.247) (width 1) (layer "F.Cu") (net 4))
 (segment (start 132 80) (end 132 94.494) (width 1) (layer "F.Cu") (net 4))
 (segment (start 140 102) (end 139.753 102.247) (width 1) (layer "F.Cu") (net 4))
 (segment (start 132.753 79.753) (end 132.5 79.5) (width 1) (layer "F.Cu") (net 4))
 (segment (start 132.5 79.5) (end 132 80) (width 1) (layer "F.Cu") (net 4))
 (segment (start 134.549 95.945) (end 134 96.494) (width 1) (layer "F.Cu") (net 4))
 (segment (start 136.055 96.945) (end 139.753 100.643) (width 1) (layer "F.Cu") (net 4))
 (segment (start 134 94) (end 134 95) (width 1) (layer "F.Cu") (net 4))
 (segment (start 134 78) (end 133 79) (width 1) (layer "F.Cu") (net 4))
 (segment (start 137.055 98.945) (end 136.753 99.247) (width 1) (layer "F.Cu") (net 4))
 (segment (start 134.11 89) (end 141.11 96) (width 1) (layer "F.Cu") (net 4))
 (segment (start 139.055 98.945) (end 137.055 98.945) (width 1) (layer "F.Cu") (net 4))
 (segment (start 141.11 96) (end 141.11 97) (width 1) (layer "F.Cu") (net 4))
 (segment (start 137.753 100.247) (end 138.753 101.247) (width 1) (layer "F.Cu") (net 4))
 (segment (start 134.11 94) (end 139.055 98.945) (width 1) (layer "F.Cu") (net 4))
 (segment (start 141.11 97) (end 141.11 98) (width 1) (layer "F.Cu") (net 4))
 (segment (start 141.11 94) (end 141.11 95) (width 1) (layer "F.Cu") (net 4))
 (segment (start 141.11 95) (end 141.11 96) (width 1) (layer "F.Cu") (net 4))
 (segment (start 134 87) (end 134.11 87) (width 1) (layer "F.Cu") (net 4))
 (segment (start 134 95) (end 134.11 95) (width 1) (layer "F.Cu") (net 4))
 (segment (start 135 87) (end 135 86) (width 1) (layer "F.Cu") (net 4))
 (segment (start 133 95) (end 132.753 95.247) (width 1) (layer "F.Cu") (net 4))
 (segment (start 134 93) (end 134 94) (width 1) (layer "F.Cu") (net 4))
 (segment (start 135 79) (end 134 78) (width 1) (layer "F.Cu") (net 4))
 (segment (start 141.11 99) (end 141.11 100) (width 1) (layer "F.Cu") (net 4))
 (segment (start 139.753 100.643) (end 139.357 100.247) (width 1) (layer "F.Cu") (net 4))
 (segment (start 134 94) (end 134.11 94) (width 1) (layer "F.Cu") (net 4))
 (segment (start 135 87) (end 141.11 93.11) (width 1) (layer "F.Cu") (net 4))
 (segment (start 132 94.494) (end 132.753 95.247) (width 1) (layer "F.Cu") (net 4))
 (segment (start 135 86) (end 135 79) (width 1) (layer "F.Cu") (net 4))
 (segment (start 134.11 87) (end 141.11 94) (width 1) (layer "F.Cu") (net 4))
 (segment (start 139.357 100.247) (end 137.753 100.247) (width 1) (layer "F.Cu") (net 4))
 (segment (start 138.753 101.247) (end 139.753 102.247) (width 1) (layer "F.Cu") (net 4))
 (segment (start 137.555 98.445) (end 141.11 102) (width 1) (layer "F.Cu") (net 4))
 (segment (start 135.055 95.945) (end 136.055 96.945) (width 1) (layer "F.Cu") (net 4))
 (segment (start 133.753 79.753) (end 133 79) (width 1) (layer "F.Cu") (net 4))
 (segment (start 134 85) (end 134 79) (width 1) (layer "F.Cu") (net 4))
 (segment (start 133.753 96.247) (end 134 96.494) (width 1) (layer "F.Cu") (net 4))
 (segment (start 134 92) (end 134 93) (width 1) (layer "F.Cu") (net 4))
 (segment (start 133 79) (end 133 95) (width 1) (layer "F.Cu") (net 4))
 (segment (start 134.11 90) (end 141.11 97) (width 1) (layer "F.Cu") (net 4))
 (segment (start 137.555 98.445) (end 137.357 98.247) (width 1) (layer "F.Cu") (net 4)))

